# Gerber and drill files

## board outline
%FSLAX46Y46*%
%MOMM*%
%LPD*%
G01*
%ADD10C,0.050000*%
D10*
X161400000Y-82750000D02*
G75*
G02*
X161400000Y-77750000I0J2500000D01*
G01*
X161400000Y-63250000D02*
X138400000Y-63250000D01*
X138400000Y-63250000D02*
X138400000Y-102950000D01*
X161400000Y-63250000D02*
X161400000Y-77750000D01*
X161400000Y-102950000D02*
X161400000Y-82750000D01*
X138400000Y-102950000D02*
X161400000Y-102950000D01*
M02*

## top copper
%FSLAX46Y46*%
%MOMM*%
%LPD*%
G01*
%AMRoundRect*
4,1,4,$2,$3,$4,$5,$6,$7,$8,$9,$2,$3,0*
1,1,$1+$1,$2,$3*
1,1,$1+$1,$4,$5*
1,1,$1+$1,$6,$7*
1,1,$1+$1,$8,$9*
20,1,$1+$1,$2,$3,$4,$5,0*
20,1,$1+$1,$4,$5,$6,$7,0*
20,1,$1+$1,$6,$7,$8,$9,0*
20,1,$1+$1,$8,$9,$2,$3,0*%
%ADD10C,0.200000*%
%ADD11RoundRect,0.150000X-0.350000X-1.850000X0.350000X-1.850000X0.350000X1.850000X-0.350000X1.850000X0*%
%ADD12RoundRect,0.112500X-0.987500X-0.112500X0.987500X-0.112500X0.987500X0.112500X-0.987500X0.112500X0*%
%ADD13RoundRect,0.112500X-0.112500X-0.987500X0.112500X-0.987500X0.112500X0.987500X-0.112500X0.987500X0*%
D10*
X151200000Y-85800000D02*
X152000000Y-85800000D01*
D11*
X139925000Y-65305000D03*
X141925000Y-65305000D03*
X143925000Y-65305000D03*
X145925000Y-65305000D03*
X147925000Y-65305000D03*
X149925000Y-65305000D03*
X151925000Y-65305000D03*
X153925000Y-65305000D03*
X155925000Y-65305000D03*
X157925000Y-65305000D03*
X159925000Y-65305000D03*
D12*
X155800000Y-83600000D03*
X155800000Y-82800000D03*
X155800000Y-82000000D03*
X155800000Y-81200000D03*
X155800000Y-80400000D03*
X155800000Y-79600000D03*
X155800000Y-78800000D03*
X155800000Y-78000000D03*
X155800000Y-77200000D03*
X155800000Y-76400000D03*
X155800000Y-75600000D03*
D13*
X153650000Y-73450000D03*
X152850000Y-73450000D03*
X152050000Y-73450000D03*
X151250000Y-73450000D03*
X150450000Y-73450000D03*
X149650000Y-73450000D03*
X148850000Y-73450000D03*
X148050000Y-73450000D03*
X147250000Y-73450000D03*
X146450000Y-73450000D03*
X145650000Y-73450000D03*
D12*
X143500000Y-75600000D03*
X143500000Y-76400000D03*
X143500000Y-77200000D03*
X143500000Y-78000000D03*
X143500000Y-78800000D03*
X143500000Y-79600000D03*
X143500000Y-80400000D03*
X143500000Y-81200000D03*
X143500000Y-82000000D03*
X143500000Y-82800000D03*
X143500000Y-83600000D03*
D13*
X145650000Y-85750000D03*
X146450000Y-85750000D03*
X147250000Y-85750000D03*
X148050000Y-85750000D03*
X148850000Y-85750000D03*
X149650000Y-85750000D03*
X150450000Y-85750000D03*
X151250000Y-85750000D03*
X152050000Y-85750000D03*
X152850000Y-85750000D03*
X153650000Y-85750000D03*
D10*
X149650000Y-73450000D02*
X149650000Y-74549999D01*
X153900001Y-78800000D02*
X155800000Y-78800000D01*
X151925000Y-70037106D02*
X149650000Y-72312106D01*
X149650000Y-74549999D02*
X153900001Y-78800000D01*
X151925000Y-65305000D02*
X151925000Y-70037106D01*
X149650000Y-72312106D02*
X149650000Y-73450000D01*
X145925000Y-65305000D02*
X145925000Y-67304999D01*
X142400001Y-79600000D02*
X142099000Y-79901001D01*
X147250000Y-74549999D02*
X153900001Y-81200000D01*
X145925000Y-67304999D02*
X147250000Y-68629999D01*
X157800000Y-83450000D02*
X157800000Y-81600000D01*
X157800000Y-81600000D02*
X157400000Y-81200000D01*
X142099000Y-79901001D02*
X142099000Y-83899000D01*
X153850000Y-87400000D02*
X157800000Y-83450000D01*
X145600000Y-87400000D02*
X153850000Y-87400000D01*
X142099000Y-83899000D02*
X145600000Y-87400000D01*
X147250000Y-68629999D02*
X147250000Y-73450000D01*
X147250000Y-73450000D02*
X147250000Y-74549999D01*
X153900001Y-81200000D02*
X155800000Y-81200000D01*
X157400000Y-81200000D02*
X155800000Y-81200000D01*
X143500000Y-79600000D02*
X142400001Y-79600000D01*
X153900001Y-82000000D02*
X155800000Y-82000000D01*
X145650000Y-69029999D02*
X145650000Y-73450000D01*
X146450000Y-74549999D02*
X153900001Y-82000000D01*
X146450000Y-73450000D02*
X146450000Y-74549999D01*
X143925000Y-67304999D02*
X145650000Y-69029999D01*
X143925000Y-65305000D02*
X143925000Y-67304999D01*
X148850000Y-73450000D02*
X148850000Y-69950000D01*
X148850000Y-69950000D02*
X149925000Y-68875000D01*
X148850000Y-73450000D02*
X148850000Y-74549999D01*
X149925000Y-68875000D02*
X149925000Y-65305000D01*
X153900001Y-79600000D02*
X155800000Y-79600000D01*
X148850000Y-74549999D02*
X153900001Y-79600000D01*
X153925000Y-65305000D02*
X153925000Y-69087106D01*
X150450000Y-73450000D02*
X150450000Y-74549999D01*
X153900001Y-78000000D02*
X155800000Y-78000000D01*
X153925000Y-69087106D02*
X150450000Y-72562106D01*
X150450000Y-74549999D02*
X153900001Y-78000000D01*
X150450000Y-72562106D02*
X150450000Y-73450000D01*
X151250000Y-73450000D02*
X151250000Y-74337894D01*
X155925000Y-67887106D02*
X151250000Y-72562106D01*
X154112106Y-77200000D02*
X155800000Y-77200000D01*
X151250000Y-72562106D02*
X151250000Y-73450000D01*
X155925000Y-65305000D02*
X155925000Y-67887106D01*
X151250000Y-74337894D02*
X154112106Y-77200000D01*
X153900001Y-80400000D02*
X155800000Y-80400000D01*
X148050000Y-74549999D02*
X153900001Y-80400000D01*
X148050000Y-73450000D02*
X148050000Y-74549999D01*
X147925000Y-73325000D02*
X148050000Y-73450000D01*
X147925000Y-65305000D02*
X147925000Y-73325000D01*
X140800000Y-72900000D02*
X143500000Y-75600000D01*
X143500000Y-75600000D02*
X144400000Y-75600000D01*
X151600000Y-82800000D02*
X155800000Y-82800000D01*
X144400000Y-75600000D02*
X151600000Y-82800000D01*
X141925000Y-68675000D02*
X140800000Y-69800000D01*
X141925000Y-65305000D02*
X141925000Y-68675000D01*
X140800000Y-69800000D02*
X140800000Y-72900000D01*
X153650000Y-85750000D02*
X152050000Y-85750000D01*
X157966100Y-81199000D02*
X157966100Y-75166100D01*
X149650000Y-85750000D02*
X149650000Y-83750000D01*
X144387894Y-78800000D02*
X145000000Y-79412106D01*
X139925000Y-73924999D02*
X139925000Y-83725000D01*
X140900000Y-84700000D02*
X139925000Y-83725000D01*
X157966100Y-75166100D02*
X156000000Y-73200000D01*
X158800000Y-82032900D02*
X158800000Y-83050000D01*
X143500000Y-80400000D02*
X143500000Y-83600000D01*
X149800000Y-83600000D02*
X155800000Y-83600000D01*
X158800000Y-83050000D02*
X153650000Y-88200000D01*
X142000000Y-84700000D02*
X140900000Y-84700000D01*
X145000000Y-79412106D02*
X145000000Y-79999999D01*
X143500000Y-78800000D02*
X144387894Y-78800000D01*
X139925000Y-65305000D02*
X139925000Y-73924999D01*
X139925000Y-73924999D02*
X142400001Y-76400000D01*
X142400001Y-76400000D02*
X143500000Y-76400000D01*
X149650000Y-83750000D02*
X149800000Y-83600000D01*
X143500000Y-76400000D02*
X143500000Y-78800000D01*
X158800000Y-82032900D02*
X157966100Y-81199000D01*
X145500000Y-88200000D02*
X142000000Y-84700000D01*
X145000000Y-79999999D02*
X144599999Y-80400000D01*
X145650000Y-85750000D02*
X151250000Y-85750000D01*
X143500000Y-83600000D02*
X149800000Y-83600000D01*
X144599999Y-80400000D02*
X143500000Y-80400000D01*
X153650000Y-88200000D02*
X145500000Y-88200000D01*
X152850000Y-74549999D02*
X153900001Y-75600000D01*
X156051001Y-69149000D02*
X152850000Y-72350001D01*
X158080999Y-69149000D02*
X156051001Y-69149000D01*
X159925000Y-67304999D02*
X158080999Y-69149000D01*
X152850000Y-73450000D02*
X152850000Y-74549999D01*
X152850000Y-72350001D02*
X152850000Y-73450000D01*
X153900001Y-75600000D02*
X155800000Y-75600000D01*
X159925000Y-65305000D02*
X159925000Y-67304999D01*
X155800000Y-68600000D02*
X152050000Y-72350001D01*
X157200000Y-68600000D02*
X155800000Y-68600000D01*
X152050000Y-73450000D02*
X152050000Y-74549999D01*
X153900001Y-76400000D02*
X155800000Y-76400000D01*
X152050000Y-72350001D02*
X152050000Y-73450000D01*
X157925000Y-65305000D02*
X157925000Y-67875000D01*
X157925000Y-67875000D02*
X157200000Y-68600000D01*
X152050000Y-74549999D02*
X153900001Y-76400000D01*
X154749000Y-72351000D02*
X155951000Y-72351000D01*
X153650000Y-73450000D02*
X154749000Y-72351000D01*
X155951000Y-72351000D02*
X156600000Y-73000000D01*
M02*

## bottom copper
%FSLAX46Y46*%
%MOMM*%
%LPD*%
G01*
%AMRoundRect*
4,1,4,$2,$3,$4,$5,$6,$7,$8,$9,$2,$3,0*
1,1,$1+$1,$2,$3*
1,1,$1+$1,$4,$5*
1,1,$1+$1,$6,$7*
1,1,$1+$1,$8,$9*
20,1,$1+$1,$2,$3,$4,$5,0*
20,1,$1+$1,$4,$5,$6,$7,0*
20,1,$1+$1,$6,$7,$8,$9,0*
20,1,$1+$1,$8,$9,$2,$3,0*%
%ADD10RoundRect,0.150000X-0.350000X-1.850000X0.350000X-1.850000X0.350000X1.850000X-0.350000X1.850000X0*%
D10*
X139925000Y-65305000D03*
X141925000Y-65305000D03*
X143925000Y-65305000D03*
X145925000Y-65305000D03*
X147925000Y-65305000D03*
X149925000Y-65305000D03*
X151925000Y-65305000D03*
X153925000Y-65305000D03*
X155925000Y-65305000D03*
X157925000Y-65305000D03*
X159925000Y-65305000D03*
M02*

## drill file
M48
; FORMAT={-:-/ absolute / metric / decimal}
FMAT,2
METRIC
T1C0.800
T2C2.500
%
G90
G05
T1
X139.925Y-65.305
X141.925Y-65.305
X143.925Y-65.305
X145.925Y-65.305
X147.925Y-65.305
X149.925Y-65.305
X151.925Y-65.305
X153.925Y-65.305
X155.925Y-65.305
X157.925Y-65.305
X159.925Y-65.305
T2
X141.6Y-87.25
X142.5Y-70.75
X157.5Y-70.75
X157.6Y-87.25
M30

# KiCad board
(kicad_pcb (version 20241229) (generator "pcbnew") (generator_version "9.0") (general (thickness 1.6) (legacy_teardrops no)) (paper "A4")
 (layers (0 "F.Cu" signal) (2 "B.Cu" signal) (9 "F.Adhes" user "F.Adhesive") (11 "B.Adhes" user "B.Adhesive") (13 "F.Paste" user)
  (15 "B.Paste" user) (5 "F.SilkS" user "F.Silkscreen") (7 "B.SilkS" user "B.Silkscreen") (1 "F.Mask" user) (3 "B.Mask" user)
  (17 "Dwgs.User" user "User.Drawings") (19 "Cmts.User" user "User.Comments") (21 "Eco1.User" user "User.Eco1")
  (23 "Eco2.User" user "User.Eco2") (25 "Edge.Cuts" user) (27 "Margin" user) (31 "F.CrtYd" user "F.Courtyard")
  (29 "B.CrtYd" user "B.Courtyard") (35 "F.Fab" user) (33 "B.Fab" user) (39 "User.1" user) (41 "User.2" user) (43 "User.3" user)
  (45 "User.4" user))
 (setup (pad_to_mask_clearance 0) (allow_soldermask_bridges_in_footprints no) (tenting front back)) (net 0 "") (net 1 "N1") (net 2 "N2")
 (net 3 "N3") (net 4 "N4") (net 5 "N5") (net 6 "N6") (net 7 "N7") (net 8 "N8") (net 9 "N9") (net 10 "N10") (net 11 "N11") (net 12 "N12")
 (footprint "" (layer "F.Cu") (at 157.5 70.75)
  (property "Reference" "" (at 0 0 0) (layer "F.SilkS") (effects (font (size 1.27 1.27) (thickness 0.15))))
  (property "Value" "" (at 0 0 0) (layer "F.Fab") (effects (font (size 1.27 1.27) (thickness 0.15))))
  (pad "" np_thru_hole circle (at 0 0) (size 2.5 2.5) (drill 2.5) (layers "*.Cu" "*.Mask")))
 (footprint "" (layer "F.Cu") (at 141.6 87.25)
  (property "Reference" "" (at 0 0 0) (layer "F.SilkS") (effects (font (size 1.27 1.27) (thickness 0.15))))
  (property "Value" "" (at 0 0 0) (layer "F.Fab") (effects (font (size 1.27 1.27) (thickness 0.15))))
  (pad "" np_thru_hole circle (at 0 0) (size 2.5 2.5) (drill 2.5) (layers "*.Cu" "*.Mask")))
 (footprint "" (layer "F.Cu") (at 142.5 70.75)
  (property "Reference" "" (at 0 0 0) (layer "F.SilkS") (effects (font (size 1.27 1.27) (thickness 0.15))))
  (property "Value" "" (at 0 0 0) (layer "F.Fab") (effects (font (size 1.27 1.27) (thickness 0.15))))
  (pad "" np_thru_hole circle (at 0 0) (size 2.5 2.5) (drill 2.5) (layers "*.Cu" "*.Mask")))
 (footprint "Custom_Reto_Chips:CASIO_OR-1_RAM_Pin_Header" (layer "F.Cu") (at 149.925 68.305)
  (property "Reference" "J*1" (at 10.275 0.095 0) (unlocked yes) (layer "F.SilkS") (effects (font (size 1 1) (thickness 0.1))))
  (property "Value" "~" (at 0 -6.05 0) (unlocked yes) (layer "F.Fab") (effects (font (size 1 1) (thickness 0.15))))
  (pad "1" thru_hole roundrect (at -10 -3) (size 1 4) (drill 0.8) (layers "*.Cu" "*.Mask") (remove_unused_layers no) (roundrect_rratio 0.15)
   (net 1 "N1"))
  (pad "2" thru_hole roundrect (at -8 -3) (size 1 4) (drill 0.8) (layers "*.Cu" "*.Mask") (remove_unused_layers no) (roundrect_rratio 0.15)
   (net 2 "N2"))
  (pad "3" thru_hole roundrect (at -6 -3) (size 1 4) (drill 0.8) (layers "*.Cu" "*.Mask") (remove_unused_layers no) (roundrect_rratio 0.15)
   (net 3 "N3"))
  (pad "4" thru_hole roundrect (at -4 -3) (size 1 4) (drill 0.8) (layers "*.Cu" "*.Mask") (remove_unused_layers no) (roundrect_rratio 0.15)
   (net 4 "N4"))
  (pad "5" thru_hole roundrect (at -2 -3) (size 1 4) (drill 0.8) (layers "*.Cu" "*.Mask") (remove_unused_layers no) (roundrect_rratio 0.15)
   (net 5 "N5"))
  (pad "6" thru_hole roundrect (at 0 -3) (size 1 4) (drill 0.8) (layers "*.Cu" "*.Mask") (remove_unused_layers no) (roundrect_rratio 0.15)
   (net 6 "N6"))
  (pad "7" thru_hole roundrect (at 2 -3) (size 1 4) (drill 0.8) (layers "*.Cu" "*.Mask") (remove_unused_layers no) (roundrect_rratio 0.15)
   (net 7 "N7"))
  (pad "8" thru_hole roundrect (at 4 -3) (size 1 4) (drill 0.8) (layers "*.Cu" "*.Mask") (remove_unused_layers no) (roundrect_rratio 0.15)
   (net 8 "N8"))
  (pad "9" thru_hole roundrect (at 6 -3) (size 1 4) (drill 0.8) (layers "*.Cu" "*.Mask") (remove_unused_layers no) (roundrect_rratio 0.15)
   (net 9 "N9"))
  (pad "10" thru_hole roundrect (at 8 -3) (size 1 4) (drill 0.8) (layers "*.Cu" "*.Mask") (remove_unused_layers no) (roundrect_rratio 0.15)
   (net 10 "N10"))
  (pad "11" thru_hole roundrect (at 10 -3) (size 1 4) (drill 0.8) (layers "*.Cu" "*.Mask") (remove_unused_layers no) (roundrect_rratio 0.15)
   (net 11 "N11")))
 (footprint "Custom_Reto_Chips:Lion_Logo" (layer "F.Cu") (at 141.6 99.8)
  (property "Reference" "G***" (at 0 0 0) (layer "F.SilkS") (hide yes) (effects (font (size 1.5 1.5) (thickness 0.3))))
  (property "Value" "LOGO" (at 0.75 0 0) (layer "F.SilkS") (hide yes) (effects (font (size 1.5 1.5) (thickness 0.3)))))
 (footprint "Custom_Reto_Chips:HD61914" (layer "F.Cu") (at 150.15 91.1)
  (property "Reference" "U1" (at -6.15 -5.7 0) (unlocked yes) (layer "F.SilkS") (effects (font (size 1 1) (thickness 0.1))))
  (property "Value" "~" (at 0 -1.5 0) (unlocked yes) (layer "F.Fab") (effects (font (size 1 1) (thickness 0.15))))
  (pad "1" smd roundrect (at 5.65 -7.5) (size 2.2 0.45) (layers "F.Cu" "F.Mask" "F.Paste") (roundrect_rratio 0.25) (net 1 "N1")
   (thermal_bridge_angle 45))
  (pad "2" smd roundrect (at 5.65 -8.3) (size 2.2 0.45) (layers "F.Cu" "F.Mask" "F.Paste") (roundrect_rratio 0.25) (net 2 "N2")
   (thermal_bridge_angle 45))
  (pad "3" smd roundrect (at 5.65 -9.1) (size 2.2 0.45) (layers "F.Cu" "F.Mask" "F.Paste") (roundrect_rratio 0.25) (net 3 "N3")
   (thermal_bridge_angle 45))
  (pad "4" smd roundrect (at 5.65 -9.9) (size 2.2 0.45) (layers "F.Cu" "F.Mask" "F.Paste") (roundrect_rratio 0.25) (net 4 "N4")
   (thermal_bridge_angle 45))
  (pad "5" smd roundrect (at 5.65 -10.7) (size 2.2 0.45) (layers "F.Cu" "F.Mask" "F.Paste") (roundrect_rratio 0.25) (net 5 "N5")
   (thermal_bridge_angle 45))
  (pad "6" smd roundrect (at 5.65 -11.5) (size 2.2 0.45) (layers "F.Cu" "F.Mask" "F.Paste") (roundrect_rratio 0.25) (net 6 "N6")
   (thermal_bridge_angle 45))
  (pad "7" smd roundrect (at 5.65 -12.3) (size 2.2 0.45) (layers "F.Cu" "F.Mask" "F.Paste") (roundrect_rratio 0.25) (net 7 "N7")
   (thermal_bridge_angle 45))
  (pad "8" smd roundrect (at 5.65 -13.1) (size 2.2 0.45) (layers "F.Cu" "F.Mask" "F.Paste") (roundrect_rratio 0.25) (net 8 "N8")
   (thermal_bridge_angle 45))
  (pad "9" smd roundrect (at 5.65 -13.9) (size 2.2 0.45) (layers "F.Cu" "F.Mask" "F.Paste") (roundrect_rratio 0.25) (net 9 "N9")
   (thermal_bridge_angle 45))
  (pad "10" smd roundrect (at 5.65 -14.7) (size 2.2 0.45) (layers "F.Cu" "F.Mask" "F.Paste") (roundrect_rratio 0.25) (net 10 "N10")
   (thermal_bridge_angle 45))
  (pad "11" smd roundrect (at 5.65 -15.5) (size 2.2 0.45) (layers "F.Cu" "F.Mask" "F.Paste") (roundrect_rratio 0.25) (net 11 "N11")
   (thermal_bridge_angle 45))
  (pad "12" smd roundrect (at 3.5 -17.65) (size 0.45 2.2) (layers "F.Cu" "F.Mask" "F.Paste") (roundrect_rratio 0.25) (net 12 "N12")
   (thermal_bridge_angle 45))
  (pad "13" smd roundrect (at 2.7 -17.65) (size 0.45 2.2) (layers "F.Cu" "F.Mask" "F.Paste") (roundrect_rratio 0.25) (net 11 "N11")
   (thermal_bridge_angle 45))
  (pad "14" smd roundrect (at 1.9 -17.65) (size 0.45 2.2) (layers "F.Cu" "F.Mask" "F.Paste") (roundrect_rratio 0.25) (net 10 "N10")
   (thermal_bridge_angle 45))
  (pad "15" smd roundrect (at 1.1 -17.65) (size 0.45 2.2) (layers "F.Cu" "F.Mask" "F.Paste") (roundrect_rratio 0.25) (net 9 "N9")
   (thermal_bridge_angle 45))
  (pad "16" smd roundrect (at 0.3 -17.65) (size 0.45 2.2) (layers "F.Cu" "F.Mask" "F.Paste") (roundrect_rratio 0.25) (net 8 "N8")
   (thermal_bridge_angle 45))
  (pad "17" smd roundrect (at -0.5 -17.65) (size 0.45 2.2) (layers "F.Cu" "F.Mask" "F.Paste") (roundrect_rratio 0.25) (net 7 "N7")
   (thermal_bridge_angle 45))
  (pad "18" smd roundrect (at -1.3 -17.65) (size 0.45 2.2) (layers "F.Cu" "F.Mask" "F.Paste") (roundrect_rratio 0.25) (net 6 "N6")
   (thermal_bridge_angle 45))
  (pad "19" smd roundrect (at -2.1 -17.65) (size 0.45 2.2) (layers "F.Cu" "F.Mask" "F.Paste") (roundrect_rratio 0.25) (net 5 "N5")
   (thermal_bridge_angle 45))
  (pad "20" smd roundrect (at -2.9 -17.65) (size 0.45 2.2) (layers "F.Cu" "F.Mask" "F.Paste") (roundrect_rratio 0.25) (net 4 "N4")
   (thermal_bridge_angle 45))
  (pad "21" smd roundrect (at -3.7 -17.65) (size 0.45 2.2) (layers "F.Cu" "F.Mask" "F.Paste") (roundrect_rratio 0.25) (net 3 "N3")
   (thermal_bridge_angle 45))
  (pad "22" smd roundrect (at -4.5 -17.65) (size 0.45 2.2) (layers "F.Cu" "F.Mask" "F.Paste") (roundrect_rratio 0.25) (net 3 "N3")
   (thermal_bridge_angle 45))
  (pad "23" smd roundrect (at -6.65 -15.5) (size 2.2 0.45) (layers "F.Cu" "F.Mask" "F.Paste") (roundrect_rratio 0.25) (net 2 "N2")
   (thermal_bridge_angle 45))
  (pad "24" smd roundrect (at -6.65 -14.7) (size 2.2 0.45) (layers "F.Cu" "F.Mask" "F.Paste") (roundrect_rratio 0.25) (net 1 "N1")
   (thermal_bridge_angle 45))
  (pad "25" smd roundrect (at -6.65 -13.9) (size 2.2 0.45) (layers "F.Cu" "F.Mask" "F.Paste") (roundrect_rratio 0.25) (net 1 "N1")
   (thermal_bridge_angle 45))
  (pad "26" smd roundrect (at -6.65 -13.1) (size 2.2 0.45) (layers "F.Cu" "F.Mask" "F.Paste") (roundrect_rratio 0.25) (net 1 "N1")
   (thermal_bridge_angle 45))
  (pad "27" smd roundrect (at -6.65 -12.3) (size 2.2 0.45) (layers "F.Cu" "F.Mask" "F.Paste") (roundrect_rratio 0.25) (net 1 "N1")
   (thermal_bridge_angle 45))
  (pad "28" smd roundrect (at -6.65 -11.5) (size 2.2 0.45) (layers "F.Cu" "F.Mask" "F.Paste") (roundrect_rratio 0.25) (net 4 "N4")
   (thermal_bridge_angle 45))
  (pad "29" smd roundrect (at -6.65 -10.7) (size 2.2 0.45) (layers "F.Cu" "F.Mask" "F.Paste") (roundrect_rratio 0.25) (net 1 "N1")
   (thermal_bridge_angle 45))
  (pad "30" smd roundrect (at -6.65 -9.9) (size 2.2 0.45) (layers "F.Cu" "F.Mask" "F.Paste") (roundrect_rratio 0.25) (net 1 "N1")
   (thermal_bridge_angle 45))
  (pad "31" smd roundrect (at -6.65 -9.1) (size 2.2 0.45) (layers "F.Cu" "F.Mask" "F.Paste") (roundrect_rratio 0.25) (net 1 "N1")
   (thermal_bridge_angle 45))
  (pad "32" smd roundrect (at -6.65 -8.3) (size 2.2 0.45) (layers "F.Cu" "F.Mask" "F.Paste") (roundrect_rratio 0.25) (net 1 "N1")
   (thermal_bridge_angle 45))
  (pad "33" smd roundrect (at -6.65 -7.5) (size 2.2 0.45) (layers "F.Cu" "F.Mask" "F.Paste") (roundrect_rratio 0.25) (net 1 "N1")
   (thermal_bridge_angle 45))
  (pad "34" smd roundrect (at -4.5 -5.35) (size 0.45 2.2) (layers "F.Cu" "F.Mask" "F.Paste") (roundrect_rratio 0.25) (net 1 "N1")
   (thermal_bridge_angle 45))
  (pad "35" smd roundrect (at -3.7 -5.35) (size 0.45 2.2) (layers "F.Cu" "F.Mask" "F.Paste") (roundrect_rratio 0.25) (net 1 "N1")
   (thermal_bridge_angle 45))
  (pad "36" smd roundrect (at -2.9 -5.35) (size 0.45 2.2) (layers "F.Cu" "F.Mask" "F.Paste") (roundrect_rratio 0.25) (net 1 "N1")
   (thermal_bridge_angle 45))
  (pad "37" smd roundrect (at -2.1 -5.35) (size 0.45 2.2) (layers "F.Cu" "F.Mask" "F.Paste") (roundrect_rratio 0.25) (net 1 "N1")
   (thermal_bridge_angle 45))
  (pad "38" smd roundrect (at -1.3 -5.35) (size 0.45 2.2) (layers "F.Cu" "F.Mask" "F.Paste") (roundrect_rratio 0.25) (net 1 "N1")
   (thermal_bridge_angle 45))
  (pad "39" smd roundrect (at -0.5 -5.35) (size 0.45 2.2) (layers "F.Cu" "F.Mask" "F.Paste") (roundrect_rratio 0.25) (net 1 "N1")
   (thermal_bridge_angle 45))
  (pad "40" smd roundrect (at 0.3 -5.35) (size 0.45 2.2) (layers "F.Cu" "F.Mask" "F.Paste") (roundrect_rratio 0.25) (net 1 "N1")
   (thermal_bridge_angle 45))
  (pad "41" smd roundrect (at 1.1 -5.35) (size 0.45 2.2) (layers "F.Cu" "F.Mask" "F.Paste") (roundrect_rratio 0.25) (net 1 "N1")
   (thermal_bridge_angle 45))
  (pad "42" smd roundrect (at 1.9 -5.35) (size 0.45 2.2) (layers "F.Cu" "F.Mask" "F.Paste") (roundrect_rratio 0.25)
   (thermal_bridge_angle 45))
  (pad "43" smd roundrect (at 2.7 -5.35) (size 0.45 2.2) (layers "F.Cu" "F.Mask" "F.Paste") (roundrect_rratio 0.25)
   (thermal_bridge_angle 45))
  (pad "44" smd roundrect (at 3.5 -5.35) (size 0.45 2.2) (layers "F.Cu" "F.Mask" "F.Paste") (roundrect_rratio 0.25)
   (thermal_bridge_angle 45)))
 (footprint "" (layer "F.Cu") (at 157.6 87.25)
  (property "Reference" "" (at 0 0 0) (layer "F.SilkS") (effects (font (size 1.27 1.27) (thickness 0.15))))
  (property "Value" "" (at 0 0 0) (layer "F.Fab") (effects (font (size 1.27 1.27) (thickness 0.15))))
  (pad "" np_thru_hole circle (at 0 0) (size 2.5 2.5) (drill 2.5) (layers "*.Cu" "*.Mask")))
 (gr_line (start 151.2 85.8) (end 152 85.8) (stroke (width 0.2) (type default)) (layer "F.Cu") (net 1))
 (gr_arc (start 161.4 82.75) (mid 158.9 80.25) (end 161.4 77.75) (stroke (width 0.05) (type default)) (layer "Edge.Cuts"))
 (gr_line (start 161.4 63.25) (end 138.4 63.25) (stroke (width 0.05) (type default)) (layer "Edge.Cuts"))
 (gr_line (start 138.4 63.25) (end 138.4 102.95) (stroke (width 0.05) (type solid)) (layer "Edge.Cuts"))
 (gr_line (start 161.4 63.25) (end 161.4 77.75) (stroke (width 0.05) (type default)) (layer "Edge.Cuts"))
 (gr_line (start 161.4 102.95) (end 161.4 82.75) (stroke (width 0.05) (type solid)) (layer "Edge.Cuts"))
 (gr_line (start 138.4 102.95) (end 161.4 102.95) (stroke (width 0.05) (type solid)) (layer "Edge.Cuts"))
 (segment (start 149.65 73.45) (end 149.65 74.549999) (width 0.2) (layer "F.Cu") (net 7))
 (segment (start 153.900001 78.8) (end 155.8 78.8) (width 0.2) (layer "F.Cu") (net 7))
 (segment (start 151.925 70.037106) (end 149.65 72.312106) (width 0.2) (layer "F.Cu") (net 7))
 (segment (start 149.65 74.549999) (end 153.900001 78.8) (width 0.2) (layer "F.Cu") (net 7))
 (segment (start 151.925 65.305) (end 151.925 70.037106) (width 0.2) (layer "F.Cu") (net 7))
 (segment (start 149.65 72.312106) (end 149.65 73.45) (width 0.2) (layer "F.Cu") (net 7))
 (segment (start 145.925 65.305) (end 145.925 67.304999) (width 0.2) (layer "F.Cu") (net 4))
 (segment (start 142.400001 79.6) (end 142.099 79.901001) (width 0.2) (layer "F.Cu") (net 4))
 (segment (start 147.25 74.549999) (end 153.900001 81.2) (width 0.2) (layer "F.Cu") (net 4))
 (segment (start 145.925 67.304999) (end 147.25 68.629999) (width 0.2) (layer "F.Cu") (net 4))
 (segment (start 157.8 83.45) (end 157.8 81.6) (width 0.2) (layer "F.Cu") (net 4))
 (segment (start 157.8 81.6) (end 157.4 81.2) (width 0.2) (layer "F.Cu") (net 4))
 (segment (start 142.099 79.901001) (end 142.099 83.899) (width 0.2) (layer "F.Cu") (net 4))
 (segment (start 153.85 87.4) (end 157.8 83.45) (width 0.2) (layer "F.Cu") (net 4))
 (segment (start 145.6 87.4) (end 153.85 87.4) (width 0.2) (layer "F.Cu") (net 4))
 (segment (start 142.099 83.899) (end 145.6 87.4) (width 0.2) (layer "F.Cu") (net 4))
 (segment (start 147.25 68.629999) (end 147.25 73.45) (width 0.2) (layer "F.Cu") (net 4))
 (segment (start 147.25 73.45) (end 147.25 74.549999) (width 0.2) (layer "F.Cu") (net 4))
 (segment (start 153.900001 81.2) (end 155.8 81.2) (width 0.2) (layer "F.Cu") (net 4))
 (segment (start 157.4 81.2) (end 155.8 81.2) (width 0.2) (layer "F.Cu") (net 4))
 (segment (start 143.5 79.6) (end 142.400001 79.6) (width 0.2) (layer "F.Cu") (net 4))
 (segment (start 153.900001 82) (end 155.8 82) (width 0.2) (layer "F.Cu") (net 3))
 (segment (start 145.65 69.029999) (end 145.65 73.45) (width 0.2) (layer "F.Cu") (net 3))
 (segment (start 146.45 74.549999) (end 153.900001 82) (width 0.2) (layer "F.Cu") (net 3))
 (segment (start 146.45 73.45) (end 146.45 74.549999) (width 0.2) (layer "F.Cu") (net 3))
 (segment (start 143.925 67.304999) (end 145.65 69.029999) (width 0.2) (layer "F.Cu") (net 3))
 (segment (start 143.925 65.305) (end 143.925 67.304999) (width 0.2) (layer "F.Cu") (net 3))
 (segment (start 148.85 73.45) (end 148.85 69.95) (width 0.2) (layer "F.Cu") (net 6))
 (segment (start 148.85 69.95) (end 149.925 68.875) (width 0.2) (layer "F.Cu") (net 6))
 (segment (start 148.85 73.45) (end 148.85 74.549999) (width 0.2) (layer "F.Cu") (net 6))
 (segment (start 149.925 68.875) (end 149.925 65.305) (width 0.2) (layer "F.Cu") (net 6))
 (segment (start 153.900001 79.6) (end 155.8 79.6) (width 0.2) (layer "F.Cu") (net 6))
 (segment (start 148.85 74.549999) (end 153.900001 79.6) (width 0.2) (layer "F.Cu") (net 6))
 (segment (start 153.925 65.305) (end 153.925 69.087106) (width 0.2) (layer "F.Cu") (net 8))
 (segment (start 150.45 73.45) (end 150.45 74.549999) (width 0.2) (layer "F.Cu") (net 8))
 (segment (start 153.900001 78) (end 155.8 78) (width 0.2) (layer "F.Cu") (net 8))
 (segment (start 153.925 69.087106) (end 150.45 72.562106) (width 0.2) (layer "F.Cu") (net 8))
 (segment (start 150.45 74.549999) (end 153.900001 78) (width 0.2) (layer "F.Cu") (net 8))
 (segment (start 150.45 72.562106) (end 150.45 73.45) (width 0.2) (layer "F.Cu") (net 8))
 (segment (start 151.25 73.45) (end 151.25 74.337894) (width 0.2) (layer "F.Cu") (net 9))
 (segment (start 155.925 67.887106) (end 151.25 72.562106) (width 0.2) (layer "F.Cu") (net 9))
 (segment (start 154.112106 77.2) (end 155.8 77.2) (width 0.2) (layer "F.Cu") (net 9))
 (segment (start 151.25 72.562106) (end 151.25 73.45) (width 0.2) (layer "F.Cu") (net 9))
 (segment (start 155.925 65.305) (end 155.925 67.887106) (width 0.2) (layer "F.Cu") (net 9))
 (segment (start 151.25 74.337894) (end 154.112106 77.2) (width 0.2) (layer "F.Cu") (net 9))
 (segment (start 153.900001 80.4) (end 155.8 80.4) (width 0.2) (layer "F.Cu") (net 5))
 (segment (start 148.05 74.549999) (end 153.900001 80.4) (width 0.2) (layer "F.Cu") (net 5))
 (segment (start 148.05 73.45) (end 148.05 74.549999) (width 0.2) (layer "F.Cu") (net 5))
 (segment (start 147.925 73.325) (end 148.05 73.45) (width 0.2) (layer "F.Cu") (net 5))
 (segment (start 147.925 65.305) (end 147.925 73.325) (width 0.2) (layer "F.Cu") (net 5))
 (segment (start 140.8 72.9) (end 143.5 75.6) (width 0.2) (layer "F.Cu") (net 2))
 (segment (start 143.5 75.6) (end 144.4 75.6) (width 0.2) (layer "F.Cu") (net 2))
 (segment (start 151.6 82.8) (end 155.8 82.8) (width 0.2) (layer "F.Cu") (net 2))
 (segment (start 144.4 75.6) (end 151.6 82.8) (width 0.2) (layer "F.Cu") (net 2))
 (segment (start 141.925 68.675) (end 140.8 69.8) (width 0.2) (layer "F.Cu") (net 2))
 (segment (start 141.925 65.305) (end 141.925 68.675) (width 0.2) (layer "F.Cu") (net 2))
 (segment (start 140.8 69.8) (end 140.8 72.9) (width 0.2) (layer "F.Cu") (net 2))
 (segment (start 153.65 85.75) (end 152.05 85.75) (width 0.2) (layer "F.Cu") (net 1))
 (segment (start 157.9661 81.199) (end 157.9661 75.1661) (width 0.2) (layer "F.Cu") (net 1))
 (segment (start 149.65 85.75) (end 149.65 83.75) (width 0.2) (layer "F.Cu") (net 1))
 (segment (start 144.387894 78.8) (end 145 79.412106) (width 0.2) (layer "F.Cu") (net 1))
 (segment (start 139.925 73.924999) (end 139.925 83.725) (width 0.2) (layer "F.Cu") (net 1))
 (segment (start 140.9 84.7) (end 139.925 83.725) (width 0.2) (layer "F.Cu") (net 1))
 (segment (start 157.9661 75.1661) (end 156 73.2) (width 0.2) (layer "F.Cu") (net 1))
 (segment (start 158.8 82.0329) (end 158.8 83.05) (width 0.2) (layer "F.Cu") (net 1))
 (segment (start 143.5 80.4) (end 143.5 83.6) (width 0.2) (layer "F.Cu") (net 1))
 (segment (start 149.8 83.6) (end 155.8 83.6) (width 0.2) (layer "F.Cu") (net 1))
 (segment (start 158.8 83.05) (end 153.65 88.2) (width 0.2) (layer "F.Cu") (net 1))
 (segment (start 142 84.7) (end 140.9 84.7) (width 0.2) (layer "F.Cu") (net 1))
 (segment (start 145 79.412106) (end 145 79.999999) (width 0.2) (layer "F.Cu") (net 1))
 (segment (start 143.5 78.8) (end 144.387894 78.8) (width 0.2) (layer "F.Cu") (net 1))
 (segment (start 139.925 65.305) (end 139.925 73.924999) (width 0.2) (layer "F.Cu") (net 1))
 (segment (start 139.925 73.924999) (end 142.400001 76.4) (width 0.2) (layer "F.Cu") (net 1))
 (segment (start 142.400001 76.4) (end 143.5 76.4) (width 0.2) (layer "F.Cu") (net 1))
 (segment (start 149.65 83.75) (end 149.8 83.6) (width 0.2) (layer "F.Cu") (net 1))
 (segment (start 143.5 76.4) (end 143.5 78.8) (width 0.2) (layer "F.Cu") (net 1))
 (segment (start 158.8 82.0329) (end 157.9661 81.199) (width 0.2) (layer "F.Cu") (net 1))
 (segment (start 145.5 88.2) (end 142 84.7) (width 0.2) (layer "F.Cu") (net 1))
 (segment (start 145 79.999999) (end 144.599999 80.4) (width 0.2) (layer "F.Cu") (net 1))
 (segment (start 145.65 85.75) (end 151.25 85.75) (width 0.2) (layer "F.Cu") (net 1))
 (segment (start 143.5 83.6) (end 149.8 83.6) (width 0.2) (layer "F.Cu") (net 1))
 (segment (start 144.599999 80.4) (end 143.5 80.4) (width 0.2) (layer "F.Cu") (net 1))
 (segment (start 153.65 88.2) (end 145.5 88.2) (width 0.2) (layer "F.Cu") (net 1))
 (segment (start 152.85 74.549999) (end 153.900001 75.6) (width 0.2) (layer "F.Cu") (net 11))
 (segment (start 156.051001 69.149) (end 152.85 72.350001) (width 0.2) (layer "F.Cu") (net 11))
 (segment (start 158.080999 69.149) (end 156.051001 69.149) (width 0.2) (layer "F.Cu") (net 11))
 (segment (start 159.925 67.304999) (end 158.080999 69.149) (width 0.2) (layer "F.Cu") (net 11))
 (segment (start 152.85 73.45) (end 152.85 74.549999) (width 0.2) (layer "F.Cu") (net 11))
 (segment (start 152.85 72.350001) (end 152.85 73.45) (width 0.2) (layer "F.Cu") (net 11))
 (segment (start 153.900001 75.6) (end 155.8 75.6) (width 0.2) (layer "F.Cu") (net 11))
 (segment (start 159.925 65.305) (end 159.925 67.304999) (width 0.2) (layer "F.Cu") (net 11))
 (segment (start 155.8 68.6) (end 152.05 72.350001) (width 0.2) (layer "F.Cu") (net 10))
 (segment (start 157.2 68.6) (end 155.8 68.6) (width 0.2) (layer "F.Cu") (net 10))
 (segment (start 152.05 73.45) (end 152.05 74.549999) (width 0.2) (layer "F.Cu") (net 10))
 (segment (start 153.900001 76.4) (end 155.8 76.4) (width 0.2) (layer "F.Cu") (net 10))
 (segment (start 152.05 72.350001) (end 152.05 73.45) (width 0.2) (layer "F.Cu") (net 10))
 (segment (start 157.925 65.305) (end 157.925 67.875) (width 0.2) (layer "F.Cu") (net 10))
 (segment (start 157.925 67.875) (end 157.2 68.6) (width 0.2) (layer "F.Cu") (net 10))
 (segment (start 152.05 74.549999) (end 153.900001 76.4) (width 0.2) (layer "F.Cu") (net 10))
 (segment (start 154.749 72.351) (end 155.951 72.351) (width 0.2) (layer "F.Cu") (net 12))
 (segment (start 153.65 73.45) (end 154.749 72.351) (width 0.2) (layer "F.Cu") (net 12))
 (segment (start 155.951 72.351) (end 156.6 73) (width 0.2) (layer "F.Cu") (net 12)))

